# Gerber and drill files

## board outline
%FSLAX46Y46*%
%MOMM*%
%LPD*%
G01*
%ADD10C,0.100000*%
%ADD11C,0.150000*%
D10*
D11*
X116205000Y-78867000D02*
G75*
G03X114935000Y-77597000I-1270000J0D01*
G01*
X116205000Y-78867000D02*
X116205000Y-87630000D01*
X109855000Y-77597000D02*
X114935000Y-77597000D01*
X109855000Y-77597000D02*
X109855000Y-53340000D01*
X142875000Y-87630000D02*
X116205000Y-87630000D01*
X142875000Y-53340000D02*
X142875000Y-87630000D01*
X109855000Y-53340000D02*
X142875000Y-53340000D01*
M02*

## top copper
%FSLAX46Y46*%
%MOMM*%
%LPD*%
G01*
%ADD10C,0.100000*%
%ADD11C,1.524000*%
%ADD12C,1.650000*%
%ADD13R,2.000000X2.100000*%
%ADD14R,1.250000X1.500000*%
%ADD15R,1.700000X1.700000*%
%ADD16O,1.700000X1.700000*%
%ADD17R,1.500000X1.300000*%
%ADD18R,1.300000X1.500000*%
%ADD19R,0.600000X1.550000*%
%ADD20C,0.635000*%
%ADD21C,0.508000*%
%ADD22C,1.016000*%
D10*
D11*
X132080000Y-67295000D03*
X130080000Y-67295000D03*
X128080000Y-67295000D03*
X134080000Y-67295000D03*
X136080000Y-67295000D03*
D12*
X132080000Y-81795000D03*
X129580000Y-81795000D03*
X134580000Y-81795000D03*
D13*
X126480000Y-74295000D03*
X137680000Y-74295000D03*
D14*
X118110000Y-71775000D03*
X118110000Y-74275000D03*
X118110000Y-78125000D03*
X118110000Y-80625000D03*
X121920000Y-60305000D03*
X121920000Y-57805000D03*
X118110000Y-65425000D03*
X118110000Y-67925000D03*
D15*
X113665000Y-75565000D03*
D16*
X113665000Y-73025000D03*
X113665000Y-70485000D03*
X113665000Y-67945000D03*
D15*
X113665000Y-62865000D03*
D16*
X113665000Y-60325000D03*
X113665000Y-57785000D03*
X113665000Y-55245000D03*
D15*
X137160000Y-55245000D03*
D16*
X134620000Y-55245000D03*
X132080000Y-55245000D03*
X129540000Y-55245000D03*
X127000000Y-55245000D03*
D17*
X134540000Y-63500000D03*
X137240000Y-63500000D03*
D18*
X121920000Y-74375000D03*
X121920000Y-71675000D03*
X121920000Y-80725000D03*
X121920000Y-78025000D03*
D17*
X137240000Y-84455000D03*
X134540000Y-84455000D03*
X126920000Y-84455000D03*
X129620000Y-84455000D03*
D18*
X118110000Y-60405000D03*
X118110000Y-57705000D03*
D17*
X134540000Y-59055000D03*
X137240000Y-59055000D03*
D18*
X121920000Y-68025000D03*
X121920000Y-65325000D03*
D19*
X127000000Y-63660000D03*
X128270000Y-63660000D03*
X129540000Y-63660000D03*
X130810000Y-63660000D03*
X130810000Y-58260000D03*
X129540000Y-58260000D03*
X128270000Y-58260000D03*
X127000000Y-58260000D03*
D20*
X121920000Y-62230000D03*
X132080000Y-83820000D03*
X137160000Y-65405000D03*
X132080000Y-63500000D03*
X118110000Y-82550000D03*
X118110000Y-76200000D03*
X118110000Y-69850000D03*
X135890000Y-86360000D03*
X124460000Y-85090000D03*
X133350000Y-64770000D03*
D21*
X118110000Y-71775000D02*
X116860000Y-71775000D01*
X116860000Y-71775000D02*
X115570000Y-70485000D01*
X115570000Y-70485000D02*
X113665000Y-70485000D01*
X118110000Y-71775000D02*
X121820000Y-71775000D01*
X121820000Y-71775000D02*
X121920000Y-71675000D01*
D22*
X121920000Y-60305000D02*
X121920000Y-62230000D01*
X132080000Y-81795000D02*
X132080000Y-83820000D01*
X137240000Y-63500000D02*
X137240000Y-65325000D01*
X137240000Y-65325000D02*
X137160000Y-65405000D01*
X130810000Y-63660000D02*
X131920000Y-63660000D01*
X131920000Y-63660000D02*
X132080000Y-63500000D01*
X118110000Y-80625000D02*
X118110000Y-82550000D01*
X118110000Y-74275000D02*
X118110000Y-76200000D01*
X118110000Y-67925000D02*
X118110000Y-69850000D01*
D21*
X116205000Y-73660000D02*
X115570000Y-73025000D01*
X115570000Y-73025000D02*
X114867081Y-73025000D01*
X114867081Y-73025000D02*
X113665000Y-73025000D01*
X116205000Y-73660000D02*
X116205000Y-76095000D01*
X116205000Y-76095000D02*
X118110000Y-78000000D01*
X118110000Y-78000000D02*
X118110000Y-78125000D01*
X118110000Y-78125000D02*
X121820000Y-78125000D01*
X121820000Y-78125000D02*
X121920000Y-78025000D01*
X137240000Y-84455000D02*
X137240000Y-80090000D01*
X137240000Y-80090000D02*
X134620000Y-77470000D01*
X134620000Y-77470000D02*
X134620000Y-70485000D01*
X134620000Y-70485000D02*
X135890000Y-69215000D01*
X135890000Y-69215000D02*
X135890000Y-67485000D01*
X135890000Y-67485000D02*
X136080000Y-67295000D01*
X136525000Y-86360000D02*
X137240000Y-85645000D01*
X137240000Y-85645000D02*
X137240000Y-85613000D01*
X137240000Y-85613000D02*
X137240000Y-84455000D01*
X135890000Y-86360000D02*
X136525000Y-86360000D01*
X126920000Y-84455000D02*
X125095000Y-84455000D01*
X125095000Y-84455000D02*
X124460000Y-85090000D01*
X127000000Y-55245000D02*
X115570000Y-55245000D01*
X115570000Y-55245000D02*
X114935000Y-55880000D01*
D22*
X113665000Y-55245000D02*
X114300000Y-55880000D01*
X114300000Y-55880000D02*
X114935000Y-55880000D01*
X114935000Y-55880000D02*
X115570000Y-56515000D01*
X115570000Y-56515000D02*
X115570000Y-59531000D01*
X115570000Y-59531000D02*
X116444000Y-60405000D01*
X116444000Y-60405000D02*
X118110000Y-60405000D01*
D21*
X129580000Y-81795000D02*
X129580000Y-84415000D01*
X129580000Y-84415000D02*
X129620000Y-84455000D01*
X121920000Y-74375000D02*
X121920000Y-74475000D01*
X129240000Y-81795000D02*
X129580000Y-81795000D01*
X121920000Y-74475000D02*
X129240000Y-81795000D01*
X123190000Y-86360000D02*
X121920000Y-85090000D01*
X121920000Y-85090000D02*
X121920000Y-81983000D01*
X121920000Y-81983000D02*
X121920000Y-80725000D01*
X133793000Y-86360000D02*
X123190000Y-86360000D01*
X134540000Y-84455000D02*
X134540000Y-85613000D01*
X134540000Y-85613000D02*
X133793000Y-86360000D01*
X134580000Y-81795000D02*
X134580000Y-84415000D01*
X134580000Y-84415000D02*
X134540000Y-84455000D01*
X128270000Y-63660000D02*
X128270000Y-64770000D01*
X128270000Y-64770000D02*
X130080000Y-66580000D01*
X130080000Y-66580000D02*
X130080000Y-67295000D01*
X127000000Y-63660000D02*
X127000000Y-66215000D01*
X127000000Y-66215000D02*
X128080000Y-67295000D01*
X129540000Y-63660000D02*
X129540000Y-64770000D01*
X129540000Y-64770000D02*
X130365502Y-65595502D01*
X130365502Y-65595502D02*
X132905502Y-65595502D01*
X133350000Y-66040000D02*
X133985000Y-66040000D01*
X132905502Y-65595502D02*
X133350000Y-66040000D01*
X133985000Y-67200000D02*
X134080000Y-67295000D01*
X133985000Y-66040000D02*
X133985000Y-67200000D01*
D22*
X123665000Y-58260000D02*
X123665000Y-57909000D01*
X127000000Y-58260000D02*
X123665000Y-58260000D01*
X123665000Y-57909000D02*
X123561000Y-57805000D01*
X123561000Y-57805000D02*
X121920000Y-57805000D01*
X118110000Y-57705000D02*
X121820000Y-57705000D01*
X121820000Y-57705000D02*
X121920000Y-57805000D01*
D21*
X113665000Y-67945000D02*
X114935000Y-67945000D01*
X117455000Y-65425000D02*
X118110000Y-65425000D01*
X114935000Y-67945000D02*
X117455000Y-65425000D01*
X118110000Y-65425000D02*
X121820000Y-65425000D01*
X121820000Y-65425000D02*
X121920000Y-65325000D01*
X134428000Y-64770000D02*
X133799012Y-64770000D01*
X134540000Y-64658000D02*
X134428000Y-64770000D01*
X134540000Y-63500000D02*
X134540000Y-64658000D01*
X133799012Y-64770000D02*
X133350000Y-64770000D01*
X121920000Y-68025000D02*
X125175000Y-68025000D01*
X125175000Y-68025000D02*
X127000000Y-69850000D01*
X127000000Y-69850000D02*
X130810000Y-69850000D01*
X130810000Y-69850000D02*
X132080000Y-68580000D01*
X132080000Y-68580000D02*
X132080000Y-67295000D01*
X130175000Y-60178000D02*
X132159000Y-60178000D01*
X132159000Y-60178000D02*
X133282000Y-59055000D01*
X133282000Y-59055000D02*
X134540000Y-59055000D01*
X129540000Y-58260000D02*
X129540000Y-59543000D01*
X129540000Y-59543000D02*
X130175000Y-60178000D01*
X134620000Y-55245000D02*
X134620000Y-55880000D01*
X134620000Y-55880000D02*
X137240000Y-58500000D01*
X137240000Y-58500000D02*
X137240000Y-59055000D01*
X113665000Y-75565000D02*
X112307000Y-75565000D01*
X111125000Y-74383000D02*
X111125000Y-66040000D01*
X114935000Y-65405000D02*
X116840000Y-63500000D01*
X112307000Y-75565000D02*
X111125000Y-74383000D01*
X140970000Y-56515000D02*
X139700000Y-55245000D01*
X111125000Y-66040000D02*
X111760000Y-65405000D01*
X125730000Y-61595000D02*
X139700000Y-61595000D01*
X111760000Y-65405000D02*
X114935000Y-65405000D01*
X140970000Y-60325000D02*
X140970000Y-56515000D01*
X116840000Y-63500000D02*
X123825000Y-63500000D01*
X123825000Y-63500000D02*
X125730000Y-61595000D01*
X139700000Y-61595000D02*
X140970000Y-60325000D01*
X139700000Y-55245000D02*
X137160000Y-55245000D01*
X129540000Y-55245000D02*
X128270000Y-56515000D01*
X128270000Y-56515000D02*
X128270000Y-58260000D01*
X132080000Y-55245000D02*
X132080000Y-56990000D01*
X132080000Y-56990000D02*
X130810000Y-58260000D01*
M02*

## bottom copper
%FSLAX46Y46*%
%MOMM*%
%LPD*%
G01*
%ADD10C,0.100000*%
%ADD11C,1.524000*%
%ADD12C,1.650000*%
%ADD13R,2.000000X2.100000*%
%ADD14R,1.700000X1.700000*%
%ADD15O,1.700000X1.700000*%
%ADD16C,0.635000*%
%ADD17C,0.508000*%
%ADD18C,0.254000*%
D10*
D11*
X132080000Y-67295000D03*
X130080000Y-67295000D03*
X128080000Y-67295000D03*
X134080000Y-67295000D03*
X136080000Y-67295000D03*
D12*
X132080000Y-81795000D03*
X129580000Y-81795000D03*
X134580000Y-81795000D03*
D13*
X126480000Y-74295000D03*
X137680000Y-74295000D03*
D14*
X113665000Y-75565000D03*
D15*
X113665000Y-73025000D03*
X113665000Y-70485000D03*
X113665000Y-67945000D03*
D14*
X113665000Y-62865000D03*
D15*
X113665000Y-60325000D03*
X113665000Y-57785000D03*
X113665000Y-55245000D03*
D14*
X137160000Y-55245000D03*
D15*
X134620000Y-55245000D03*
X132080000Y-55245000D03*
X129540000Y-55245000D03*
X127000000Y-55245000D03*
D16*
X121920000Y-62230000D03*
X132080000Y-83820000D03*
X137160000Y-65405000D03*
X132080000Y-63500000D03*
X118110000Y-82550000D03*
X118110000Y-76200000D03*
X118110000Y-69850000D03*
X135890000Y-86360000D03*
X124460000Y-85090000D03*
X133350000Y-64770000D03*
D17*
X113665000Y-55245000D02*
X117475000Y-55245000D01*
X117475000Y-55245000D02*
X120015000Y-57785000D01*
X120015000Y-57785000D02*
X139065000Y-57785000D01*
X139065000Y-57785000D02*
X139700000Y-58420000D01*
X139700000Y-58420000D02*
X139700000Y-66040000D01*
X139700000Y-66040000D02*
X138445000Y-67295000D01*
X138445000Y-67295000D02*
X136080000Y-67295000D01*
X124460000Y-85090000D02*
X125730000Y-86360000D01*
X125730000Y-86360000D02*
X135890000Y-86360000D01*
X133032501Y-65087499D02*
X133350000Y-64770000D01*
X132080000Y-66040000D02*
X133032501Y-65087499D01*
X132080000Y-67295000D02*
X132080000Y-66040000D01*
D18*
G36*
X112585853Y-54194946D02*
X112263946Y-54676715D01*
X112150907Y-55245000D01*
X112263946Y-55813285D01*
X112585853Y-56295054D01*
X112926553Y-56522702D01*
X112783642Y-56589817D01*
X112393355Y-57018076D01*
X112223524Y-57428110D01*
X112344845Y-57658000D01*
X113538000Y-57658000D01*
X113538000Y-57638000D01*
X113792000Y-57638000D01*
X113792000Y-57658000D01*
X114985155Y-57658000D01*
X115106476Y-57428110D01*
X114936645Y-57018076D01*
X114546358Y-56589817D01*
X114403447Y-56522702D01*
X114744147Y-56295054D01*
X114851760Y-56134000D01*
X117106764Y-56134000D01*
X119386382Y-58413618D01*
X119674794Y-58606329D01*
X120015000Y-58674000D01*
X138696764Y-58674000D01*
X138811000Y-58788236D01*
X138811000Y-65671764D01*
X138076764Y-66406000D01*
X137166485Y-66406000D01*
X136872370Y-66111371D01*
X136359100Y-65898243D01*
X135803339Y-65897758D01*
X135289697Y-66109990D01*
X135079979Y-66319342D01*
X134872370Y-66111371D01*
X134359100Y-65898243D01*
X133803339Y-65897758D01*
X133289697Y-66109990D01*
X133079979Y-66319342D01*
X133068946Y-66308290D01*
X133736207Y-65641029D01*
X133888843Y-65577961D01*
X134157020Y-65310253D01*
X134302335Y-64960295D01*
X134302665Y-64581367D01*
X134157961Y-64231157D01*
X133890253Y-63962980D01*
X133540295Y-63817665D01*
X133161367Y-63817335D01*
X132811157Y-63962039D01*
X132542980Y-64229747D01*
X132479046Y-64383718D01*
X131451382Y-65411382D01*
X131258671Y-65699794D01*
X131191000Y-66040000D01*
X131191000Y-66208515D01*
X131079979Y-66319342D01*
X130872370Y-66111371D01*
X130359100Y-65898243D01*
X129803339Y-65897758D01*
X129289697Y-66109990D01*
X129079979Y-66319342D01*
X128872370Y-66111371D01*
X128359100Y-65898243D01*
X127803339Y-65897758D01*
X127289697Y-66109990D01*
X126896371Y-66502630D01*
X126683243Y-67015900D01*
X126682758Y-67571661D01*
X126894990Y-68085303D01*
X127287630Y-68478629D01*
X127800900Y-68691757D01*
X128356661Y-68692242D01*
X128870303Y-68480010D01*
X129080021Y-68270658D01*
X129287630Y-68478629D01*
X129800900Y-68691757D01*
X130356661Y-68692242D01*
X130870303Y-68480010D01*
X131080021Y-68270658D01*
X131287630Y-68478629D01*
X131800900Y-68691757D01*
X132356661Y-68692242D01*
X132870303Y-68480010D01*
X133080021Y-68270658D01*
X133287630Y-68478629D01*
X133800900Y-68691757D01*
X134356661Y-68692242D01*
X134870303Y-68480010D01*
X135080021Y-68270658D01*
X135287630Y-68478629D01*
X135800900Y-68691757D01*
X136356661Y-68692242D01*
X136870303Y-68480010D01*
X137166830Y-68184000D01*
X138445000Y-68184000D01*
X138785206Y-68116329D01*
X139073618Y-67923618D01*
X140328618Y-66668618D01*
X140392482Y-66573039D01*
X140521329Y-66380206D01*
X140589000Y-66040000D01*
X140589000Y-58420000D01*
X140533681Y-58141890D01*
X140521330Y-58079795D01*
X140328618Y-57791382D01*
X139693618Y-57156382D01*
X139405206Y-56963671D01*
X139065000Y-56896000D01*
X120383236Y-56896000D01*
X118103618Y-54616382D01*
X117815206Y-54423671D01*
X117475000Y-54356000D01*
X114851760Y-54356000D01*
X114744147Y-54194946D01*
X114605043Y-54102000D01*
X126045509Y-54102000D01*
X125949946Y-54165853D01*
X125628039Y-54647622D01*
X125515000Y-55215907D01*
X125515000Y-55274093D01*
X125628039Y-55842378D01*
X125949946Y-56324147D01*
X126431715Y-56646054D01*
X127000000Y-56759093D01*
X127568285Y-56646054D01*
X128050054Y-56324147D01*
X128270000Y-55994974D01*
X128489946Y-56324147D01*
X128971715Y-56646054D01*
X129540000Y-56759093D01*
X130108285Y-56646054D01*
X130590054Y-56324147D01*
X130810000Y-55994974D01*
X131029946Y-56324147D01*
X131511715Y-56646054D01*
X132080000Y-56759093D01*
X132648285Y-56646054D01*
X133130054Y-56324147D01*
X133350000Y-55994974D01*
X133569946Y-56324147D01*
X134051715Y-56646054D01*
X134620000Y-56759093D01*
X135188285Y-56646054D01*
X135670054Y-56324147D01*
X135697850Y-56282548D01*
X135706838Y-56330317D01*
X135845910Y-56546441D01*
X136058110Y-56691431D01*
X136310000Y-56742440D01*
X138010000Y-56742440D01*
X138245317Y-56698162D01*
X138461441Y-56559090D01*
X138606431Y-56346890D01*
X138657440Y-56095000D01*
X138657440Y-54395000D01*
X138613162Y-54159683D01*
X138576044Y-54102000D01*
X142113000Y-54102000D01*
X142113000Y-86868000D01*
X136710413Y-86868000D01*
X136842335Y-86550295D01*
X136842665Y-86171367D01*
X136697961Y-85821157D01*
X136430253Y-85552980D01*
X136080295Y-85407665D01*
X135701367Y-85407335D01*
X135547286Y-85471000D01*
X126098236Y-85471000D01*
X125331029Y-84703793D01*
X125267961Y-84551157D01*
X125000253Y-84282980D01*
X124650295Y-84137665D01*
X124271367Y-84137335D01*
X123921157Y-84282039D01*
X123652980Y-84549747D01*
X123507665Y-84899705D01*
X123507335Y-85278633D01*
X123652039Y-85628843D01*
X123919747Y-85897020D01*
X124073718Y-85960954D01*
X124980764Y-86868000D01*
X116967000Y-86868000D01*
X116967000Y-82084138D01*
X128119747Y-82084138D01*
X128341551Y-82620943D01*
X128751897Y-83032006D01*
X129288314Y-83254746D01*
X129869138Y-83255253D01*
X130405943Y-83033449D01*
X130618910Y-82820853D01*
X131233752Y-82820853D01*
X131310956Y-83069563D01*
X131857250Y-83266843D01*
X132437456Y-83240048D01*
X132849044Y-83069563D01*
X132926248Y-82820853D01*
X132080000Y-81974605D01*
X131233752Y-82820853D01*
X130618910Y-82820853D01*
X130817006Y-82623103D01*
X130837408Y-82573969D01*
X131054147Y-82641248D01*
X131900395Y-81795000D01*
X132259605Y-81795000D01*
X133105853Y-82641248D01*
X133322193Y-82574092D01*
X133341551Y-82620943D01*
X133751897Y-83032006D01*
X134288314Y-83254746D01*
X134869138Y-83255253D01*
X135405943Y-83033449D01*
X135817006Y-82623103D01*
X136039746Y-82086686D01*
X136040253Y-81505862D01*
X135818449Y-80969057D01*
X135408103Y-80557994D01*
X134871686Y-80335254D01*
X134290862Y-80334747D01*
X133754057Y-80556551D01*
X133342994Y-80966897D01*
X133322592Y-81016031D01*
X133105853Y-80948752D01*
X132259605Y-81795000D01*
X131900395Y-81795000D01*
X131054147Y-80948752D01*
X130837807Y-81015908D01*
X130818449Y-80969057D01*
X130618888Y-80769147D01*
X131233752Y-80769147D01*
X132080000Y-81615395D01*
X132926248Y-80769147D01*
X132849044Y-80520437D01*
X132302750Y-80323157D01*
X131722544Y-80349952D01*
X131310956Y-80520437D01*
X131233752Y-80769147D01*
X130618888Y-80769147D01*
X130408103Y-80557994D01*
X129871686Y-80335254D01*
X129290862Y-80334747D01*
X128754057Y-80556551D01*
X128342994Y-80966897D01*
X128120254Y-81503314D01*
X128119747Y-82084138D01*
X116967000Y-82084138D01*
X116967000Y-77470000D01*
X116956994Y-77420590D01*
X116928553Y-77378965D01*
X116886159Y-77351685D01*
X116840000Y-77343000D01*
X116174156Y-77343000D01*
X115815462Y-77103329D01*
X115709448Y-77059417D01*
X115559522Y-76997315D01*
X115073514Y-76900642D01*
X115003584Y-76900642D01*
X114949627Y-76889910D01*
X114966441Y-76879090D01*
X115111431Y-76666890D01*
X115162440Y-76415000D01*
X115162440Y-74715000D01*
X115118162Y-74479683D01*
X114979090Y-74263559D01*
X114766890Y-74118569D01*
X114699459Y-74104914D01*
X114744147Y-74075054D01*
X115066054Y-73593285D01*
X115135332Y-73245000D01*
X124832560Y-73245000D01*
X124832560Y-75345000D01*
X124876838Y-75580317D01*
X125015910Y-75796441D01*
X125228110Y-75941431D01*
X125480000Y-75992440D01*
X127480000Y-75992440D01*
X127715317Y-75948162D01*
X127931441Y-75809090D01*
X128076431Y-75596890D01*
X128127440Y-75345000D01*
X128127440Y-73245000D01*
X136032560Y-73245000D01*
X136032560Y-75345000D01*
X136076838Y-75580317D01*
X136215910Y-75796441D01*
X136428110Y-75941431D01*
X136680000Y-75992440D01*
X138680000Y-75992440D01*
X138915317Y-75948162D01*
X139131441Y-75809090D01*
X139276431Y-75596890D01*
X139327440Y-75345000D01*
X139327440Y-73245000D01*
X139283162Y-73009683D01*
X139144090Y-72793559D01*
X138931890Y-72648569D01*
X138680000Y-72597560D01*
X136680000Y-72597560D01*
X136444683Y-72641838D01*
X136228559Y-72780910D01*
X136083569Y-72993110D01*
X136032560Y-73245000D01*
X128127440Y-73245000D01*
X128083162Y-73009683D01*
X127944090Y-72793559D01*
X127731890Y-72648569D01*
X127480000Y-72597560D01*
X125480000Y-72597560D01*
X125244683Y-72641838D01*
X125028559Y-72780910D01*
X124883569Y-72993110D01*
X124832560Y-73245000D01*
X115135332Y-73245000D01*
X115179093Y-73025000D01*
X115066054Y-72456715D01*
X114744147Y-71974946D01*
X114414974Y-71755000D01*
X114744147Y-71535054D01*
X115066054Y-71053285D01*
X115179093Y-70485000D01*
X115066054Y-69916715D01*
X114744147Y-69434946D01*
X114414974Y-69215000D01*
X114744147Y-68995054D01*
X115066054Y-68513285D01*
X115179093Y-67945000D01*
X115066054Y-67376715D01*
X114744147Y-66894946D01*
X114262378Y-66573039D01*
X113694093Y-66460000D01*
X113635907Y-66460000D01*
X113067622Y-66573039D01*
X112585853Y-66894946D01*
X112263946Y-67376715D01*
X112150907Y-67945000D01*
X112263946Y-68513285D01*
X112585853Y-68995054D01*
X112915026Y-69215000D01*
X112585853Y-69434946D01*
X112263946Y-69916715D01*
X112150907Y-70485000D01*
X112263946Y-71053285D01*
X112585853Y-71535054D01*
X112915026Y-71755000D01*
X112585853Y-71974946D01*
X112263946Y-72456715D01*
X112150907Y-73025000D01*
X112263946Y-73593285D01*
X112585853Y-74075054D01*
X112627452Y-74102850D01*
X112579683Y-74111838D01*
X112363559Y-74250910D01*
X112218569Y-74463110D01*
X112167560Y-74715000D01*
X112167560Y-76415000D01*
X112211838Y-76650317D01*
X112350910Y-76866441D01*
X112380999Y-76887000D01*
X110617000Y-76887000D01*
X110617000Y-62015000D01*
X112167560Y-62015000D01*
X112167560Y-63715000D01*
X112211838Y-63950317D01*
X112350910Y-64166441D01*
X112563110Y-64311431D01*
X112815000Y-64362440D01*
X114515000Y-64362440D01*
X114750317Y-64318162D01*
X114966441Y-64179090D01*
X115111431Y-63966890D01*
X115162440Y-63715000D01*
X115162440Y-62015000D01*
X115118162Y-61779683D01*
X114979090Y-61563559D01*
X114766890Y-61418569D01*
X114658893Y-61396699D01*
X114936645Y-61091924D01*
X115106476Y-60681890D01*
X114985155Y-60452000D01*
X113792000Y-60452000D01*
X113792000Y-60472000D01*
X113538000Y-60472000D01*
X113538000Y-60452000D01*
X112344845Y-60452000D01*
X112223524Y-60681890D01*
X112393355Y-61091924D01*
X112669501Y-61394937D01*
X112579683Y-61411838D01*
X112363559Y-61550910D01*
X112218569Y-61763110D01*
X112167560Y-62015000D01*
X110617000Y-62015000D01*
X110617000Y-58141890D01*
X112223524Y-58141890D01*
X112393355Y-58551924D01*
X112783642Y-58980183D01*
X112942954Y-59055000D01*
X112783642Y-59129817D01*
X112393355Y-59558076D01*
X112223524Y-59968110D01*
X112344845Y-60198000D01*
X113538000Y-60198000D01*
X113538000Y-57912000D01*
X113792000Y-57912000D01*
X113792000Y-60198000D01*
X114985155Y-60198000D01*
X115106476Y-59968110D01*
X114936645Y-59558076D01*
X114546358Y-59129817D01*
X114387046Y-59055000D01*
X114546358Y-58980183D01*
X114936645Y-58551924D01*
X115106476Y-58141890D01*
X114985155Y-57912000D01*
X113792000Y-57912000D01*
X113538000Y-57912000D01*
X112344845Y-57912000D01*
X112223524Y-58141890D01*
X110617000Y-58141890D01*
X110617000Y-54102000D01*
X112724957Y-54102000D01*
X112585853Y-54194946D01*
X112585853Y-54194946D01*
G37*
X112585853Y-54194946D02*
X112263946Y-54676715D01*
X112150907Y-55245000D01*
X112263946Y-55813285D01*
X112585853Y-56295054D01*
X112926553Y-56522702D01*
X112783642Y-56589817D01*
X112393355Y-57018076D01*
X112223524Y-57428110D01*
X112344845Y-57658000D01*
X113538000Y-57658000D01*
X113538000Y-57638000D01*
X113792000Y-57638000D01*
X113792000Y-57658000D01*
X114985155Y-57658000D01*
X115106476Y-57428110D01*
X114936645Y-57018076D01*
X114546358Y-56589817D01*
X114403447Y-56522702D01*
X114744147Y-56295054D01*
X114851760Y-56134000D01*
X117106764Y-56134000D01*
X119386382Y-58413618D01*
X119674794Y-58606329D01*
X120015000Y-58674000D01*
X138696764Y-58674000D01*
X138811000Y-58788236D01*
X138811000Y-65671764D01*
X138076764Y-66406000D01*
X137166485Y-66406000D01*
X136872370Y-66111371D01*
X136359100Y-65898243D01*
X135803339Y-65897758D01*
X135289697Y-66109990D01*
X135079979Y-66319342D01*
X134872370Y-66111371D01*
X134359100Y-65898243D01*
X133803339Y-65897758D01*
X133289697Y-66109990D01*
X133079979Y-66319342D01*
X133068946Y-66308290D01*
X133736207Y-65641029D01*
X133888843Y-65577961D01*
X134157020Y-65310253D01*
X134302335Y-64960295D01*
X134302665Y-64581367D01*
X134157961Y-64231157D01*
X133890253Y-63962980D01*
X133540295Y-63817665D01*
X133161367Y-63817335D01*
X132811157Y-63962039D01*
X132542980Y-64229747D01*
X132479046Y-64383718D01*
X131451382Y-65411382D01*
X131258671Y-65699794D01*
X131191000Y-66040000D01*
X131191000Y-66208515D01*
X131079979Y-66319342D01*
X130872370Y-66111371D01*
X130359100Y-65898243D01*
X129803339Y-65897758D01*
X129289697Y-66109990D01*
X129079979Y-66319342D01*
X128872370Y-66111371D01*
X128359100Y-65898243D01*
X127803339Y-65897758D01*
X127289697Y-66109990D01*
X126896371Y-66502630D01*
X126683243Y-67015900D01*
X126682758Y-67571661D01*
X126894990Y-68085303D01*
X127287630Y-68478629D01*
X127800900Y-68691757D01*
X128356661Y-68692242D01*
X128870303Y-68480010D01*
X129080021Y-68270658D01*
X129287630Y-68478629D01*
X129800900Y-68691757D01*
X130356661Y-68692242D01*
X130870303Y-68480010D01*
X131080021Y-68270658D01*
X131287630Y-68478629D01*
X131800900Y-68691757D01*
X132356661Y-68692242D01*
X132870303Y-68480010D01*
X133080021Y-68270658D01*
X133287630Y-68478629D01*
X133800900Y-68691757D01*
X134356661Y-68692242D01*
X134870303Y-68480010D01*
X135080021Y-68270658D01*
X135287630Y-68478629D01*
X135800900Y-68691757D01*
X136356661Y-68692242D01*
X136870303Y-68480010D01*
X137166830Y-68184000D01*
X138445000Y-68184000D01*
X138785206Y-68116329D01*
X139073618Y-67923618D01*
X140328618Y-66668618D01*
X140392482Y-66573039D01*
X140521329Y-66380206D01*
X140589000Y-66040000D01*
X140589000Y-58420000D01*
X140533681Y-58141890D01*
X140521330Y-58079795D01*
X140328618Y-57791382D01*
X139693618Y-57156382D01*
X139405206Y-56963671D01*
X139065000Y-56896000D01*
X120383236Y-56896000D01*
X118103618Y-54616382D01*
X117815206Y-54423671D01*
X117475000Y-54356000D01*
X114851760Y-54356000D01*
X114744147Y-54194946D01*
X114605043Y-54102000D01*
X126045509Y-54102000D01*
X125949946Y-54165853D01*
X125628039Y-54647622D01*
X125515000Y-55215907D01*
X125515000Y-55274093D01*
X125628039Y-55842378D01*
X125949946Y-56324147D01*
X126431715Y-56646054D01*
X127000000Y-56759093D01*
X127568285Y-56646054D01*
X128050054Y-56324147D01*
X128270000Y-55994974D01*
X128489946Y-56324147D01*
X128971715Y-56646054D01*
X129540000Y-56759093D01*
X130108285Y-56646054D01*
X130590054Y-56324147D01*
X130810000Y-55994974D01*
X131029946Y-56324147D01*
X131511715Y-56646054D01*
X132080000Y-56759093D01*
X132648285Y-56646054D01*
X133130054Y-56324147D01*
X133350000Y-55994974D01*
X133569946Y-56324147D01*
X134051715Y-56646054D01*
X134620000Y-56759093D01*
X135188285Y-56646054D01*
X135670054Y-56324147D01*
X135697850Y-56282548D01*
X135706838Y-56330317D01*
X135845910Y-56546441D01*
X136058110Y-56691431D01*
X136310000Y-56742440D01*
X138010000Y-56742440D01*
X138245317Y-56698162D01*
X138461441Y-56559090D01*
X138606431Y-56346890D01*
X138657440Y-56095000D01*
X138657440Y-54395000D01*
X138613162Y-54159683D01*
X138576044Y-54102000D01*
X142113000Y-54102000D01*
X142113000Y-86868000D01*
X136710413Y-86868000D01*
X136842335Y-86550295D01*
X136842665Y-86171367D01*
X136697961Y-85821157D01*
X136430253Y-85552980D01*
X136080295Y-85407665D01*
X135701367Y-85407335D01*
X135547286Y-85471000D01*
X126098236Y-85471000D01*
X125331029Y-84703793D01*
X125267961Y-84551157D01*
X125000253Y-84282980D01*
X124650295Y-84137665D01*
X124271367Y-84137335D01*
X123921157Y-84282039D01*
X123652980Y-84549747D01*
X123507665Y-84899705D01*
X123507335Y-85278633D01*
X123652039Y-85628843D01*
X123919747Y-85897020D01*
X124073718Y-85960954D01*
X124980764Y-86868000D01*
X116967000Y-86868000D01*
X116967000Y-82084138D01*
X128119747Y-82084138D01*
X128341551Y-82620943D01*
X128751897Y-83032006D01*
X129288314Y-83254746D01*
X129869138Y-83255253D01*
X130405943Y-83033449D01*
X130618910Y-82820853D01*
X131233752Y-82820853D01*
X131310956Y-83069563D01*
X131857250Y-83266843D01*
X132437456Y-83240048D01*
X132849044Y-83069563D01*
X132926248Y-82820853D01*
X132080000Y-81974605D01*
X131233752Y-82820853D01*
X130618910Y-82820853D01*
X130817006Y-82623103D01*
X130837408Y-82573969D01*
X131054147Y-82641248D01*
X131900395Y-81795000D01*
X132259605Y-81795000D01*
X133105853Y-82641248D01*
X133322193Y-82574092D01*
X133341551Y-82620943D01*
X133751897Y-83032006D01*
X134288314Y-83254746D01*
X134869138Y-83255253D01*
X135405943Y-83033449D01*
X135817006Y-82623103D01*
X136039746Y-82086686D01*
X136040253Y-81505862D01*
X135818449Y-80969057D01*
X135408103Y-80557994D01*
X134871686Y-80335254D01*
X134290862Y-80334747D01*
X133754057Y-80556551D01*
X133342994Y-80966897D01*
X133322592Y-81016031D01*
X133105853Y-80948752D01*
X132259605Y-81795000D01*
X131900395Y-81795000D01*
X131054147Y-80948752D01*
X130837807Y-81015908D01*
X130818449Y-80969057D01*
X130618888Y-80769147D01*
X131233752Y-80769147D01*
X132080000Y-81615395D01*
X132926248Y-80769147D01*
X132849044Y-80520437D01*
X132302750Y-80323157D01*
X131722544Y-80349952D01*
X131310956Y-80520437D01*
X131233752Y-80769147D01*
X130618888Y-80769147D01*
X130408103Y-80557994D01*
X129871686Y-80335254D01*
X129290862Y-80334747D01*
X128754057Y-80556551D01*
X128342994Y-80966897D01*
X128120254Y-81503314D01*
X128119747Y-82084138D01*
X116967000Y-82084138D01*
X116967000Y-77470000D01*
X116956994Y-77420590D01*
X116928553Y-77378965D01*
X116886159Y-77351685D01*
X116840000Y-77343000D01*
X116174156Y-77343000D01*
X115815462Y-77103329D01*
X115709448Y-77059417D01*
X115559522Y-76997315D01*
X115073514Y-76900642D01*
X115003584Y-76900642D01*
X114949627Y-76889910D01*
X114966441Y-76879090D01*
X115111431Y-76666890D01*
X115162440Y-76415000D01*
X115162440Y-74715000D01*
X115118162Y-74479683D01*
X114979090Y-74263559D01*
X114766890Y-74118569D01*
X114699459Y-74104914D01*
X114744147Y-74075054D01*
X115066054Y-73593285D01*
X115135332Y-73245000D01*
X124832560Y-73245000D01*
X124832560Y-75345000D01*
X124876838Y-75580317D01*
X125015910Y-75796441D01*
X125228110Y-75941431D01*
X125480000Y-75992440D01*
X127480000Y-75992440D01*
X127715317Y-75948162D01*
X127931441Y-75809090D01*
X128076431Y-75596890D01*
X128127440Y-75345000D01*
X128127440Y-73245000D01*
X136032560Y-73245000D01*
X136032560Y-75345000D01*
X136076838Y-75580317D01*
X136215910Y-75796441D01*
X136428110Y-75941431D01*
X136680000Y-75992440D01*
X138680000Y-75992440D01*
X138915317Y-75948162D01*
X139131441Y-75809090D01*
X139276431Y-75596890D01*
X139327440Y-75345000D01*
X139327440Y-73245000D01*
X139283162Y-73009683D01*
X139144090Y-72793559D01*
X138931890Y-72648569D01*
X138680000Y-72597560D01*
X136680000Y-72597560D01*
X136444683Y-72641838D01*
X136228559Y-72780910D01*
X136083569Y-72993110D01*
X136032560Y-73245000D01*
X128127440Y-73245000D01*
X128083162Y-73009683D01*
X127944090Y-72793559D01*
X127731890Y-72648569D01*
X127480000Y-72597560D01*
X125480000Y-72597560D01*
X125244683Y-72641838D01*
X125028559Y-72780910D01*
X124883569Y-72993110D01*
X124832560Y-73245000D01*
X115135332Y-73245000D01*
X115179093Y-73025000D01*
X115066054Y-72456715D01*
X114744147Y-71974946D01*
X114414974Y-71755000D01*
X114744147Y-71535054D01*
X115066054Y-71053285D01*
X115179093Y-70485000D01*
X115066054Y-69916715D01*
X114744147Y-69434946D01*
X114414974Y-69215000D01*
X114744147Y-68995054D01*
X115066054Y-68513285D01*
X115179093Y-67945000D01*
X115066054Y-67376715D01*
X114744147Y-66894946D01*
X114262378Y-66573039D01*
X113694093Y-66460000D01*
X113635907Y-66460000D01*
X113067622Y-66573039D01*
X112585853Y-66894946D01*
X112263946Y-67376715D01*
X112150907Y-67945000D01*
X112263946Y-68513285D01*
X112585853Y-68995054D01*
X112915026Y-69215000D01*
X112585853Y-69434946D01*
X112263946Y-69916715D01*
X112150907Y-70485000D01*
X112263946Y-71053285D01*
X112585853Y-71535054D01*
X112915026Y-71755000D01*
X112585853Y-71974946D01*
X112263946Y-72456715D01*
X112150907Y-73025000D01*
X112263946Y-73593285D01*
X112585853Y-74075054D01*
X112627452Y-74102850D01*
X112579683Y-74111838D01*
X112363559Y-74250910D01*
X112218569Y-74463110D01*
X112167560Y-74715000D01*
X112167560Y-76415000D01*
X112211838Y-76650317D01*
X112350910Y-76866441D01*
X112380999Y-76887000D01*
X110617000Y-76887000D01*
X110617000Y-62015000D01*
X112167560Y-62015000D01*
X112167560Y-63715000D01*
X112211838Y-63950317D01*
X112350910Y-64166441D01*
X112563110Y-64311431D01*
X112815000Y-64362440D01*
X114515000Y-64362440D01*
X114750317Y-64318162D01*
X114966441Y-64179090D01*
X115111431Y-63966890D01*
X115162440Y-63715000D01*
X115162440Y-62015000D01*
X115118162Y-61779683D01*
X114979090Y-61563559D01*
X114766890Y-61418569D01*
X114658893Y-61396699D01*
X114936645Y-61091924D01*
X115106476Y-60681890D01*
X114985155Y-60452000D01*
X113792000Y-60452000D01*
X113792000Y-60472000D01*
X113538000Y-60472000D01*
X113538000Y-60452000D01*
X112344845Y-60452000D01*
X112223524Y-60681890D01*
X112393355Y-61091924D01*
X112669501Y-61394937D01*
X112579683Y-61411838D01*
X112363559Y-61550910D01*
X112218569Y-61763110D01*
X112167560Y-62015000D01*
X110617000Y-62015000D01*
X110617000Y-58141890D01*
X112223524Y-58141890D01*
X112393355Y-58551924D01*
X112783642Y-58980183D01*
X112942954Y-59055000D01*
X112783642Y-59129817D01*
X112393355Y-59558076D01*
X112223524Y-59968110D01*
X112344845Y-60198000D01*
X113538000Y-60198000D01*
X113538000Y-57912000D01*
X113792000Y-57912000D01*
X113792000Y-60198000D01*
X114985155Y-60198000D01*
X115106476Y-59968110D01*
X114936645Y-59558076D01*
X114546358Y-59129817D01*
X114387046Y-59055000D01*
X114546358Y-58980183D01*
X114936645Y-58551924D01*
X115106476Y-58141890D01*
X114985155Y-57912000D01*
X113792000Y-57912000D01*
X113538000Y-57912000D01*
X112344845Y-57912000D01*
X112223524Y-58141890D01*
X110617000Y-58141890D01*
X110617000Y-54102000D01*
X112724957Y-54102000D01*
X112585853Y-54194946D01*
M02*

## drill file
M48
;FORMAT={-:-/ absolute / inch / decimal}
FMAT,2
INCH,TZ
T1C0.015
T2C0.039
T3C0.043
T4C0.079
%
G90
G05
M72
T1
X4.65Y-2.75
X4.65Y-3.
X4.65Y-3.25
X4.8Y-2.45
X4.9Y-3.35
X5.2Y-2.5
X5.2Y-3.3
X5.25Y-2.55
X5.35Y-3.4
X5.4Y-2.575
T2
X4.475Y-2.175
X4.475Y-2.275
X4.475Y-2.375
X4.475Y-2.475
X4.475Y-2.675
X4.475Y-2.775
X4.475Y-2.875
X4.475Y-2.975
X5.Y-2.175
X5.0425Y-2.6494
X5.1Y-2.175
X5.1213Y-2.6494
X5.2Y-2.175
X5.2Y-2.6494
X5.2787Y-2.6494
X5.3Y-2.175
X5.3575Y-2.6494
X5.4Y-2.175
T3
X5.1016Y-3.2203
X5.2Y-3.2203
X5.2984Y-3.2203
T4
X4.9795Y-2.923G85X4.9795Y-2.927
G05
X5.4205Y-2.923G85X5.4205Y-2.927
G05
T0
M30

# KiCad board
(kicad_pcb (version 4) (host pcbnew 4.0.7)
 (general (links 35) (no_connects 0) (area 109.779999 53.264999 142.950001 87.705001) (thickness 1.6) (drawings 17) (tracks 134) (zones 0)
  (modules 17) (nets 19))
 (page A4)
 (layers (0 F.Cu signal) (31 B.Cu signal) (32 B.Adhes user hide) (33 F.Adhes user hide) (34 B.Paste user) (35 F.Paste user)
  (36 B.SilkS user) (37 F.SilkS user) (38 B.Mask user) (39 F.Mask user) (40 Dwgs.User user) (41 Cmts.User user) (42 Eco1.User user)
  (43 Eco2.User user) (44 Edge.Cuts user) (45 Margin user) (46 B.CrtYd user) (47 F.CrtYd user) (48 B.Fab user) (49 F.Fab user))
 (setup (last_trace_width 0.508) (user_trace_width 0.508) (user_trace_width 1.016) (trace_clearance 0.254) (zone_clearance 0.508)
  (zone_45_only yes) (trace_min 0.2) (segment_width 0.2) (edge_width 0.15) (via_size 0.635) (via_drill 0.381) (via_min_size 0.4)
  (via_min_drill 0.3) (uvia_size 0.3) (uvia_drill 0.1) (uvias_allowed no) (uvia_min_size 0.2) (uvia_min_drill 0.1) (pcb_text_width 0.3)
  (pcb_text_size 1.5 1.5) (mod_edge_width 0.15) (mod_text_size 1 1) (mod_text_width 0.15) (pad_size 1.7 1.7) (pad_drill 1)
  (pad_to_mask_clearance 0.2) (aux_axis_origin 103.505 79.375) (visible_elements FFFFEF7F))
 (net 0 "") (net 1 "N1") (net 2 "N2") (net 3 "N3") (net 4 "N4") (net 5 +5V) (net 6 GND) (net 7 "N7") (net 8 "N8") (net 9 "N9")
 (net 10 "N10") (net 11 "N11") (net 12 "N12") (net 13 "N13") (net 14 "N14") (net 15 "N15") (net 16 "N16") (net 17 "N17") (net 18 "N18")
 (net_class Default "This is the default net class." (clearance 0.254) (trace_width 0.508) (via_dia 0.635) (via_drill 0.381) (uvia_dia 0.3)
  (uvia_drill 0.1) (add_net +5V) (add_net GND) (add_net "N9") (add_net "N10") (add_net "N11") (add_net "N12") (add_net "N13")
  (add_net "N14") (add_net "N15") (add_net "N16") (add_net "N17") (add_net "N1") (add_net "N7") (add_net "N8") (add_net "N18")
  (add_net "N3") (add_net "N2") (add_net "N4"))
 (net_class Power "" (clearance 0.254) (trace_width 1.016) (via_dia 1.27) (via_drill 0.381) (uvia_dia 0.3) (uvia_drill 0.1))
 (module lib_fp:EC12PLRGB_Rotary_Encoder (layer F.Cu) (at 132.08 74.295)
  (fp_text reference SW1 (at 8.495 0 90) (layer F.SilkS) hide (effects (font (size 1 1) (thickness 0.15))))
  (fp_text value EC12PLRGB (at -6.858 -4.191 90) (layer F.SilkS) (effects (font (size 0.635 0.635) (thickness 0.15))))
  (pad 3 thru_hole circle (at 0 -7) (size 1.524 1.524) (drill 1) (layers *.Cu *.Mask) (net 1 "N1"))
  (pad 2 thru_hole circle (at -2 -7) (size 1.524 1.524) (drill 1) (layers *.Cu *.Mask) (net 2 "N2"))
  (pad 1 thru_hole circle (at -4 -7) (size 1.524 1.524) (drill 1) (layers *.Cu *.Mask) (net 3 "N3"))
  (pad 4 thru_hole circle (at 2 -7) (size 1.524 1.524) (drill 1) (layers *.Cu *.Mask) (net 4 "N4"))
  (pad 5 thru_hole circle (at 4 -7) (size 1.524 1.524) (drill 1) (layers *.Cu *.Mask) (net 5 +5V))
  (pad C thru_hole circle (at 0 7.5) (size 1.65 1.65) (drill 1.1) (layers *.Cu *.Mask) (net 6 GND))
  (pad A thru_hole circle (at -2.5 7.5) (size 1.65 1.65) (drill 1.1) (layers *.Cu *.Mask) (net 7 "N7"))
  (pad B thru_hole circle (at 2.5 7.5) (size 1.65 1.65) (drill 1.1) (layers *.Cu *.Mask) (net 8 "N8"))
  (pad "" np_thru_hole rect (at -5.6 0) (size 2 2.1) (drill oval 2 2.1) (layers *.Cu *.Mask))
  (pad "" np_thru_hole rect (at 5.6 0) (size 2 2.1) (drill oval 2 2.1) (layers *.Cu *.Mask)))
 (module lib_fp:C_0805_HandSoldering (layer F.Cu) (at 118.11 73.025 270)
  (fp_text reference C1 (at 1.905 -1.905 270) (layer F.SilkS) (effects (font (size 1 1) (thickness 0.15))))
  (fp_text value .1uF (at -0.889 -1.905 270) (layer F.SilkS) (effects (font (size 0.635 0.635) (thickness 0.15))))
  (pad 1 smd rect (at -1.25 0 270) (size 1.5 1.25) (layers F.Cu F.Paste F.Mask) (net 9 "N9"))
  (pad 2 smd rect (at 1.25 0 270) (size 1.5 1.25) (layers F.Cu F.Paste F.Mask) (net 6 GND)))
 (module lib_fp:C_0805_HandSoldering (layer F.Cu) (at 118.11 79.375 270)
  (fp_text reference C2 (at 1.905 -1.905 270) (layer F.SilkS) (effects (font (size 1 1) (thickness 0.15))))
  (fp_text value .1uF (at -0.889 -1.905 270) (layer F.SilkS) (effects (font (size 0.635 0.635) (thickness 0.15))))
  (pad 1 smd rect (at -1.25 0 270) (size 1.5 1.25) (layers F.Cu F.Paste F.Mask) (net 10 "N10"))
  (pad 2 smd rect (at 1.25 0 270) (size 1.5 1.25) (layers F.Cu F.Paste F.Mask) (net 6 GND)))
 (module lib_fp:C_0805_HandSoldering (layer F.Cu) (at 121.92 59.055 90)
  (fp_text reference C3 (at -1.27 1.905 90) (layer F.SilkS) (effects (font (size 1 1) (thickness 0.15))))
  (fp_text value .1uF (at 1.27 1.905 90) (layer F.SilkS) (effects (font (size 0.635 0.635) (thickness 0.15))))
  (pad 1 smd rect (at -1.25 0 90) (size 1.5 1.25) (layers F.Cu F.Paste F.Mask) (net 6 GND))
  (pad 2 smd rect (at 1.25 0 90) (size 1.5 1.25) (layers F.Cu F.Paste F.Mask) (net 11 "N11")))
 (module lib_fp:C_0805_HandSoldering (layer F.Cu) (at 118.11 66.675 270)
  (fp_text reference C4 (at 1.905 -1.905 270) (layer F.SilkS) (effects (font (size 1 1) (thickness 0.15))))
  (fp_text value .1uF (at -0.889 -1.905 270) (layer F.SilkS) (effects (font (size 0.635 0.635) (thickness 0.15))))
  (pad 1 smd rect (at -1.25 0 270) (size 1.5 1.25) (layers F.Cu F.Paste F.Mask) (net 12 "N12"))
  (pad 2 smd rect (at 1.25 0 270) (size 1.5 1.25) (layers F.Cu F.Paste F.Mask) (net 6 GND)))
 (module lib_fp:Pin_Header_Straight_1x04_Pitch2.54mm (layer B.Cu) (at 113.665 75.565)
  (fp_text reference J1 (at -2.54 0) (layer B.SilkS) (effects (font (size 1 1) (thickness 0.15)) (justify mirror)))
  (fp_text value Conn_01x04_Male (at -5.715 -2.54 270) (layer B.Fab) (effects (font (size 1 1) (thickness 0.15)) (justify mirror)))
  (pad 1 thru_hole rect (at 0 0) (size 1.7 1.7) (drill 1) (layers *.Cu *.Mask) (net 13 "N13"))
  (pad 2 thru_hole oval (at 0 -2.54) (size 1.7 1.7) (drill 1) (layers *.Cu *.Mask) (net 10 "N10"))
  (pad 3 thru_hole oval (at 0 -5.08) (size 1.7 1.7) (drill 1) (layers *.Cu *.Mask) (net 9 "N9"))
  (pad 4 thru_hole oval (at 0 -7.62) (size 1.7 1.7) (drill 1) (layers *.Cu *.Mask) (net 12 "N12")))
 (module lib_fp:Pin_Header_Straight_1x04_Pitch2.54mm (layer B.Cu) (at 113.665 62.865)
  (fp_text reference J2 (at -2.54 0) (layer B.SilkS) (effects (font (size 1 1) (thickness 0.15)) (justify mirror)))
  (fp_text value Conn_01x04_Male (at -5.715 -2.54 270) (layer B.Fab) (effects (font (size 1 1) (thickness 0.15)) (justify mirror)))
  (pad 1 thru_hole rect (at 0 0) (size 1.7 1.7) (drill 1) (layers *.Cu *.Mask) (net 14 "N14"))
  (pad 2 thru_hole oval (at 0 -2.54) (size 1.7 1.7) (drill 1) (layers *.Cu *.Mask) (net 6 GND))
  (pad 3 thru_hole oval (at 0 -5.08) (size 1.7 1.7) (drill 1) (layers *.Cu *.Mask) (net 6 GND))
  (pad 4 thru_hole oval (at 0 -7.62) (size 1.7 1.7) (drill 1) (layers *.Cu *.Mask) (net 5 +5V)))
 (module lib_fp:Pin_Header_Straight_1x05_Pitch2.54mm (layer F.Cu) (at 137.16 55.245 270)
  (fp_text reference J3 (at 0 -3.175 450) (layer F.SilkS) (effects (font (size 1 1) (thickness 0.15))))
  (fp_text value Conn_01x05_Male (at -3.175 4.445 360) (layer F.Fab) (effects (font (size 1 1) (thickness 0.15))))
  (pad 1 thru_hole rect (at 0 0 270) (size 1.7 1.7) (drill 1) (layers *.Cu *.Mask) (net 13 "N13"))
  (pad 2 thru_hole oval (at 0 2.54 270) (size 1.7 1.7) (drill 1) (layers *.Cu *.Mask) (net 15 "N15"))
  (pad 3 thru_hole oval (at 0 5.08 270) (size 1.7 1.7) (drill 1) (layers *.Cu *.Mask) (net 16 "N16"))
  (pad 4 thru_hole oval (at 0 7.62 270) (size 1.7 1.7) (drill 1) (layers *.Cu *.Mask) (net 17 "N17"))
  (pad 5 thru_hole oval (at 0 10.16 270) (size 1.7 1.7) (drill 1) (layers *.Cu *.Mask) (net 5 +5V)))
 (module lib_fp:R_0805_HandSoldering (layer F.Cu) (at 135.89 63.5)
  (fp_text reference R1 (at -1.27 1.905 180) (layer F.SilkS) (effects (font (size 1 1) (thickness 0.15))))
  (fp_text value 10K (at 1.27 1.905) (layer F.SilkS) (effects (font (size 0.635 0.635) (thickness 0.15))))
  (pad 1 smd rect (at -1.35 0) (size 1.5 1.3) (layers F.Cu F.Paste F.Mask) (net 1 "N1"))
  (pad 2 smd rect (at 1.35 0) (size 1.5 1.3) (layers F.Cu F.Paste F.Mask) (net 6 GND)))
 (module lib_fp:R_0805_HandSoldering (layer F.Cu) (at 121.92 73.025 90)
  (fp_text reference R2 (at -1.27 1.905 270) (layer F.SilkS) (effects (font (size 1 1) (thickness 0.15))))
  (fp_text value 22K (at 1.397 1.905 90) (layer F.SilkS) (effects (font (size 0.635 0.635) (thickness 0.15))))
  (pad 1 smd rect (at -1.35 0 90) (size 1.5 1.3) (layers F.Cu F.Paste F.Mask) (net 7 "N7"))
  (pad 2 smd rect (at 1.35 0 90) (size 1.5 1.3) (layers F.Cu F.Paste F.Mask) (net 9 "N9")))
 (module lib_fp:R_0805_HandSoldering (layer F.Cu) (at 121.92 79.375 90)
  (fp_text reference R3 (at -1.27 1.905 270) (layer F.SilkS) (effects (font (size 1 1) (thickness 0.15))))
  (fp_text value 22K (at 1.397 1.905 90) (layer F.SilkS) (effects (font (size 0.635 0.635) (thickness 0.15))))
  (pad 1 smd rect (at -1.35 0 90) (size 1.5 1.3) (layers F.Cu F.Paste F.Mask) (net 8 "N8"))
  (pad 2 smd rect (at 1.35 0 90) (size 1.5 1.3) (layers F.Cu F.Paste F.Mask) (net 10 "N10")))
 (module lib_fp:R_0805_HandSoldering (layer F.Cu) (at 135.89 84.455 180)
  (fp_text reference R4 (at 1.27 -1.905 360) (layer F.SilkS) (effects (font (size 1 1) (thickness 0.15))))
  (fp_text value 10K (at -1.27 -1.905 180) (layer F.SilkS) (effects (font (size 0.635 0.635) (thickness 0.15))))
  (pad 1 smd rect (at -1.35 0 180) (size 1.5 1.3) (layers F.Cu F.Paste F.Mask) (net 5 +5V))
  (pad 2 smd rect (at 1.35 0 180) (size 1.5 1.3) (layers F.Cu F.Paste F.Mask) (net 8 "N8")))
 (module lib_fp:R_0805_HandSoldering (layer F.Cu) (at 128.27 84.455)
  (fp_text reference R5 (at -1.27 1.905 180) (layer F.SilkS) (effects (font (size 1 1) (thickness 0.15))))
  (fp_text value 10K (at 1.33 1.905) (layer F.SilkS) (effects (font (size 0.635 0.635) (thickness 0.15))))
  (pad 1 smd rect (at -1.35 0) (size 1.5 1.3) (layers F.Cu F.Paste F.Mask) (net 5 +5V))
  (pad 2 smd rect (at 1.35 0) (size 1.5 1.3) (layers F.Cu F.Paste F.Mask) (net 7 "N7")))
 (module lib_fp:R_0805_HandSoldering (layer F.Cu) (at 118.11 59.055 90)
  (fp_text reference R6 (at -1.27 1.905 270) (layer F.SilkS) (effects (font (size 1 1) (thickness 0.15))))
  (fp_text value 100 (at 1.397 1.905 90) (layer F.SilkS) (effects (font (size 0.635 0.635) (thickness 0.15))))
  (pad 1 smd rect (at -1.35 0 90) (size 1.5 1.3) (layers F.Cu F.Paste F.Mask) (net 5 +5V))
  (pad 2 smd rect (at 1.35 0 90) (size 1.5 1.3) (layers F.Cu F.Paste F.Mask) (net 11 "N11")))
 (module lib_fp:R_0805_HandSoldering (layer F.Cu) (at 135.89 59.055)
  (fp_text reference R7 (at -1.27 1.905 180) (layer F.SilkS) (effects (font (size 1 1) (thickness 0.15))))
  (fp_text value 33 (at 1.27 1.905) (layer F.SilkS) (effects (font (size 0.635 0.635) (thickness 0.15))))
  (pad 1 smd rect (at -1.35 0) (size 1.5 1.3) (layers F.Cu F.Paste F.Mask) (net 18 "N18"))
  (pad 2 smd rect (at 1.35 0) (size 1.5 1.3) (layers F.Cu F.Paste F.Mask) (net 15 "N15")))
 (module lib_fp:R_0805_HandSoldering (layer F.Cu) (at 121.92 66.675 90)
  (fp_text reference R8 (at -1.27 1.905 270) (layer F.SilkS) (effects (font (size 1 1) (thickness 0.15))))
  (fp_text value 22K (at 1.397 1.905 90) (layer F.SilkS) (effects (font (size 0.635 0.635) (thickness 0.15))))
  (pad 1 smd rect (at -1.35 0 90) (size 1.5 1.3) (layers F.Cu F.Paste F.Mask) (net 1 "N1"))
  (pad 2 smd rect (at 1.35 0 90) (size 1.5 1.3) (layers F.Cu F.Paste F.Mask) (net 12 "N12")))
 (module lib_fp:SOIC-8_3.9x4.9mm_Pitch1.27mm (layer F.Cu) (at 128.905 60.96 90)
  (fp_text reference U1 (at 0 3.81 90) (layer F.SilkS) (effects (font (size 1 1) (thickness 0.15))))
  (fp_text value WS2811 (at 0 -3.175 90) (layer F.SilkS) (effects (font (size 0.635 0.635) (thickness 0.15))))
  (pad 1 smd rect (at -2.7 -1.905 90) (size 1.55 0.6) (layers F.Cu F.Paste F.Mask) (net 3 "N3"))
  (pad 2 smd rect (at -2.7 -0.635 90) (size 1.55 0.6) (layers F.Cu F.Paste F.Mask) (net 2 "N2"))
  (pad 3 smd rect (at -2.7 0.635 90) (size 1.55 0.6) (layers F.Cu F.Paste F.Mask) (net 4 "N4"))
  (pad 4 smd rect (at -2.7 1.905 90) (size 1.55 0.6) (layers F.Cu F.Paste F.Mask) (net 6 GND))
  (pad 5 smd rect (at 2.7 1.905 90) (size 1.55 0.6) (layers F.Cu F.Paste F.Mask) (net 16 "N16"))
  (pad 6 smd rect (at 2.7 0.635 90) (size 1.55 0.6) (layers F.Cu F.Paste F.Mask) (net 18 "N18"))
  (pad 7 smd rect (at 2.7 -0.635 90) (size 1.55 0.6) (layers F.Cu F.Paste F.Mask) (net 17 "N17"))
  (pad 8 smd rect (at 2.7 -1.905 90) (size 1.55 0.6) (layers F.Cu F.Paste F.Mask) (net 11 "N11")))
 (gr_arc (start 114.935 78.867) (end 114.935 77.597) (angle 90) (layer Edge.Cuts) (width 0.15))
 (gr_line (start 116.205 78.867) (end 116.205 87.63) (layer Edge.Cuts) (width 0.15))
 (gr_line (start 109.855 77.597) (end 114.935 77.597) (layer Edge.Cuts) (width 0.15))
 (gr_line (start 109.855 77.597) (end 109.855 53.34) (layer Edge.Cuts) (width 0.15))
 (gr_line (start 142.875 87.63) (end 116.205 87.63) (layer Edge.Cuts) (width 0.15))
 (gr_line (start 142.875 53.34) (end 142.875 87.63) (layer Edge.Cuts) (width 0.15))
 (gr_line (start 109.855 53.34) (end 142.875 53.34) (layer Edge.Cuts) (width 0.15))
 (segment (start 118.11 71.775) (end 116.86 71.775) (width 0.508) (layer F.Cu) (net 9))
 (segment (start 116.86 71.775) (end 115.57 70.485) (width 0.508) (layer F.Cu) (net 9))
 (segment (start 115.57 70.485) (end 113.665 70.485) (width 0.508) (layer F.Cu) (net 9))
 (segment (start 118.11 71.775) (end 121.82 71.775) (width 0.508) (layer F.Cu) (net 9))
 (segment (start 121.82 71.775) (end 121.92 71.675) (width 0.508) (layer F.Cu) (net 9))
 (segment (start 121.92 60.305) (end 121.92 62.23) (width 1.016) (layer F.Cu) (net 6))
 (via (at 121.92 62.23) (size 0.635) (drill 0.381) (layers F.Cu B.Cu) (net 6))
 (segment (start 132.08 81.795) (end 132.08 83.82) (width 1.016) (layer F.Cu) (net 6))
 (via (at 132.08 83.82) (size 0.635) (drill 0.381) (layers F.Cu B.Cu) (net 6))
 (segment (start 137.24 63.5) (end 137.24 65.325) (width 1.016) (layer F.Cu) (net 6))
 (segment (start 137.24 65.325) (end 137.16 65.405) (width 1.016) (layer F.Cu) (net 6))
 (via (at 137.16 65.405) (size 0.635) (drill 0.381) (layers F.Cu B.Cu) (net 6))
 (segment (start 130.81 63.66) (end 131.92 63.66) (width 1.016) (layer F.Cu) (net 6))
 (segment (start 131.92 63.66) (end 132.08 63.5) (width 1.016) (layer F.Cu) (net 6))
 (via (at 132.08 63.5) (size 0.635) (drill 0.381) (layers F.Cu B.Cu) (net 6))
 (segment (start 118.11 80.625) (end 118.11 82.55) (width 1.016) (layer F.Cu) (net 6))
 (via (at 118.11 82.55) (size 0.635) (drill 0.381) (layers F.Cu B.Cu) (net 6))
 (segment (start 118.11 74.275) (end 118.11 76.2) (width 1.016) (layer F.Cu) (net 6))
 (via (at 118.11 76.2) (size 0.635) (drill 0.381) (layers F.Cu B.Cu) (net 6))
 (via (at 118.11 69.85) (size 0.635) (drill 0.381) (layers F.Cu B.Cu) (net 6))
 (segment (start 118.11 67.925) (end 118.11 69.85) (width 1.016) (layer F.Cu) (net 6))
 (segment (start 116.205 73.66) (end 115.57 73.025) (width 0.508) (layer F.Cu) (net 10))
 (segment (start 115.57 73.025) (end 114.867081 73.025) (width 0.508) (layer F.Cu) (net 10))
 (segment (start 114.867081 73.025) (end 113.665 73.025) (width 0.508) (layer F.Cu) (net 10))
 (segment (start 116.205 73.66) (end 116.205 76.095) (width 0.508) (layer F.Cu) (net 10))
 (segment (start 116.205 76.095) (end 118.11 78) (width 0.508) (layer F.Cu) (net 10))
 (segment (start 118.11 78) (end 118.11 78.125) (width 0.508) (layer F.Cu) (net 10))
 (segment (start 118.11 78.125) (end 121.82 78.125) (width 0.508) (layer F.Cu) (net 10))
 (segment (start 121.82 78.125) (end 121.92 78.025) (width 0.508) (layer F.Cu) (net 10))
 (segment (start 137.24 84.455) (end 137.24 80.09) (width 0.508) (layer F.Cu) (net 5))
 (segment (start 137.24 80.09) (end 134.62 77.47) (width 0.508) (layer F.Cu) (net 5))
 (segment (start 134.62 77.47) (end 134.62 70.485) (width 0.508) (layer F.Cu) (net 5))
 (segment (start 134.62 70.485) (end 135.89 69.215) (width 0.508) (layer F.Cu) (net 5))
 (segment (start 135.89 69.215) (end 135.89 67.485) (width 0.508) (layer F.Cu) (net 5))
 (segment (start 135.89 67.485) (end 136.08 67.295) (width 0.508) (layer F.Cu) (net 5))
 (segment (start 113.665 55.245) (end 117.475 55.245) (width 0.508) (layer B.Cu) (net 5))
 (segment (start 117.475 55.245) (end 120.015 57.785) (width 0.508) (layer B.Cu) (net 5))
 (segment (start 120.015 57.785) (end 139.065 57.785) (width 0.508) (layer B.Cu) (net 5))
 (segment (start 139.065 57.785) (end 139.7 58.42) (width 0.508) (layer B.Cu) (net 5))
 (segment (start 139.7 58.42) (end 139.7 66.04) (width 0.508) (layer B.Cu) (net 5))
 (segment (start 139.7 66.04) (end 138.445 67.295) (width 0.508) (layer B.Cu) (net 5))
 (segment (start 138.445 67.295) (end 136.08 67.295) (width 0.508) (layer B.Cu) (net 5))
 (segment (start 136.525 86.36) (end 137.24 85.645) (width 0.508) (layer F.Cu) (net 5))
 (segment (start 137.24 85.645) (end 137.24 85.613) (width 0.508) (layer F.Cu) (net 5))
 (segment (start 137.24 85.613) (end 137.24 84.455) (width 0.508) (layer F.Cu) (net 5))
 (segment (start 135.89 86.36) (end 136.525 86.36) (width 0.508) (layer F.Cu) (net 5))
 (segment (start 124.46 85.09) (end 125.73 86.36) (width 0.508) (layer B.Cu) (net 5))
 (segment (start 125.73 86.36) (end 135.89 86.36) (width 0.508) (layer B.Cu) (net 5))
 (via (at 135.89 86.36) (size 0.635) (drill 0.381) (layers F.Cu B.Cu) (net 5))
 (segment (start 126.92 84.455) (end 125.095 84.455) (width 0.508) (layer F.Cu) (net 5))
 (segment (start 125.095 84.455) (end 124.46 85.09) (width 0.508) (layer F.Cu) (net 5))
 (via (at 124.46 85.09) (size 0.635) (drill 0.381) (layers F.Cu B.Cu) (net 5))
 (segment (start 127 55.245) (end 115.57 55.245) (width 0.508) (layer F.Cu) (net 5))
 (segment (start 115.57 55.245) (end 114.935 55.88) (width 0.508) (layer F.Cu) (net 5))
 (segment (start 113.665 55.245) (end 114.3 55.88) (width 1.016) (layer F.Cu) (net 5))
 (segment (start 114.3 55.88) (end 114.935 55.88) (width 1.016) (layer F.Cu) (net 5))
 (segment (start 114.935 55.88) (end 115.57 56.515) (width 1.016) (layer F.Cu) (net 5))
 (segment (start 115.57 56.515) (end 115.57 59.531) (width 1.016) (layer F.Cu) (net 5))
 (segment (start 115.57 59.531) (end 116.444 60.405) (width 1.016) (layer F.Cu) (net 5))
 (segment (start 116.444 60.405) (end 118.11 60.405) (width 1.016) (layer F.Cu) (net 5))
 (segment (start 129.58 81.795) (end 129.58 84.415) (width 0.508) (layer F.Cu) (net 7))
 (segment (start 129.58 84.415) (end 129.62 84.455) (width 0.508) (layer F.Cu) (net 7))
 (segment (start 121.92 74.375) (end 121.92 74.475) (width 0.508) (layer F.Cu) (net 7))
 (segment (start 129.24 81.795) (end 129.58 81.795) (width 0.508) (layer F.Cu) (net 7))
 (segment (start 121.92 74.475) (end 129.24 81.795) (width 0.508) (layer F.Cu) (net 7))
 (segment (start 123.19 86.36) (end 121.92 85.09) (width 0.508) (layer F.Cu) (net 8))
 (segment (start 121.92 85.09) (end 121.92 81.983) (width 0.508) (layer F.Cu) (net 8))
 (segment (start 121.92 81.983) (end 121.92 80.725) (width 0.508) (layer F.Cu) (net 8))
 (segment (start 133.793 86.36) (end 123.19 86.36) (width 0.508) (layer F.Cu) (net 8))
 (segment (start 134.54 84.455) (end 134.54 85.613) (width 0.508) (layer F.Cu) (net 8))
 (segment (start 134.54 85.613) (end 133.793 86.36) (width 0.508) (layer F.Cu) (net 8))
 (segment (start 134.58 81.795) (end 134.58 84.415) (width 0.508) (layer F.Cu) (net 8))
 (segment (start 134.58 84.415) (end 134.54 84.455) (width 0.508) (layer F.Cu) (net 8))
 (segment (start 128.27 63.66) (end 128.27 64.77) (width 0.508) (layer F.Cu) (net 2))
 (segment (start 128.27 64.77) (end 130.08 66.58) (width 0.508) (layer F.Cu) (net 2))
 (segment (start 130.08 66.58) (end 130.08 67.295) (width 0.508) (layer F.Cu) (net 2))
 (segment (start 127 63.66) (end 127 66.215) (width 0.508) (layer F.Cu) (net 3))
 (segment (start 127 66.215) (end 128.08 67.295) (width 0.508) (layer F.Cu) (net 3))
 (segment (start 129.54 63.66) (end 129.54 64.77) (width 0.508) (layer F.Cu) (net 4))
 (segment (start 129.54 64.77) (end 130.365502 65.595502) (width 0.508) (layer F.Cu) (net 4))
 (segment (start 130.365502 65.595502) (end 132.905502 65.595502) (width 0.508) (layer F.Cu) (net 4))
 (segment (start 133.35 66.04) (end 133.985 66.04) (width 0.508) (layer F.Cu) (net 4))
 (segment (start 132.905502 65.595502) (end 133.35 66.04) (width 0.508) (layer F.Cu) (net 4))
 (segment (start 133.985 67.2) (end 134.08 67.295) (width 0.508) (layer F.Cu) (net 4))
 (segment (start 133.985 66.04) (end 133.985 67.2) (width 0.508) (layer F.Cu) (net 4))
 (segment (start 123.665 58.26) (end 123.665 57.909) (width 1.016) (layer F.Cu) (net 11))
 (segment (start 127 58.26) (end 123.665 58.26) (width 1.016) (layer F.Cu) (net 11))
 (segment (start 123.665 57.909) (end 123.561 57.805) (width 1.016) (layer F.Cu) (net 11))
 (segment (start 123.561 57.805) (end 121.92 57.805) (width 1.016) (layer F.Cu) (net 11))
 (segment (start 118.11 57.705) (end 121.82 57.705) (width 1.016) (layer F.Cu) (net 11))
 (segment (start 121.82 57.705) (end 121.92 57.805) (width 1.016) (layer F.Cu) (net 11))
 (segment (start 113.665 67.945) (end 114.935 67.945) (width 0.508) (layer F.Cu) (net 12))
 (segment (start 117.455 65.425) (end 118.11 65.425) (width 0.508) (layer F.Cu) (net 12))
 (segment (start 114.935 67.945) (end 117.455 65.425) (width 0.508) (layer F.Cu) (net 12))
 (segment (start 118.11 65.425) (end 121.82 65.425) (width 0.508) (layer F.Cu) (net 12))
 (segment (start 121.82 65.425) (end 121.92 65.325) (width 0.508) (layer F.Cu) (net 12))
 (segment (start 133.032501 65.087499) (end 133.35 64.77) (width 0.508) (layer B.Cu) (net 1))
 (segment (start 132.08 66.04) (end 133.032501 65.087499) (width 0.508) (layer B.Cu) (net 1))
 (segment (start 132.08 67.295) (end 132.08 66.04) (width 0.508) (layer B.Cu) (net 1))
 (segment (start 134.428 64.77) (end 133.799012 64.77) (width 0.508) (layer F.Cu) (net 1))
 (segment (start 134.54 64.658) (end 134.428 64.77) (width 0.508) (layer F.Cu) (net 1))
 (segment (start 134.54 63.5) (end 134.54 64.658) (width 0.508) (layer F.Cu) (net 1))
 (segment (start 133.799012 64.77) (end 133.35 64.77) (width 0.508) (layer F.Cu) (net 1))
 (via (at 133.35 64.77) (size 0.635) (drill 0.381) (layers F.Cu B.Cu) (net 1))
 (segment (start 121.92 68.025) (end 125.175 68.025) (width 0.508) (layer F.Cu) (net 1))
 (segment (start 125.175 68.025) (end 127 69.85) (width 0.508) (layer F.Cu) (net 1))
 (segment (start 127 69.85) (end 130.81 69.85) (width 0.508) (layer F.Cu) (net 1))
 (segment (start 130.81 69.85) (end 132.08 68.58) (width 0.508) (layer F.Cu) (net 1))
 (segment (start 132.08 68.58) (end 132.08 67.295) (width 0.508) (layer F.Cu) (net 1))
 (segment (start 130.175 60.178) (end 132.159 60.178) (width 0.508) (layer F.Cu) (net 18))
 (segment (start 132.159 60.178) (end 133.282 59.055) (width 0.508) (layer F.Cu) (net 18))
 (segment (start 133.282 59.055) (end 134.54 59.055) (width 0.508) (layer F.Cu) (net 18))
 (segment (start 129.54 58.26) (end 129.54 59.543) (width 0.508) (layer F.Cu) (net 18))
 (segment (start 129.54 59.543) (end 130.175 60.178) (width 0.508) (layer F.Cu) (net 18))
 (segment (start 134.62 55.245) (end 134.62 55.88) (width 0.508) (layer F.Cu) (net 15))
 (segment (start 134.62 55.88) (end 137.24 58.5) (width 0.508) (layer F.Cu) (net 15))
 (segment (start 137.24 58.5) (end 137.24 59.055) (width 0.508) (layer F.Cu) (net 15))
 (segment (start 113.665 75.565) (end 112.307 75.565) (width 0.508) (layer F.Cu) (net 13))
 (segment (start 111.125 74.383) (end 111.125 66.04) (width 0.508) (layer F.Cu) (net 13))
 (segment (start 114.935 65.405) (end 116.84 63.5) (width 0.508) (layer F.Cu) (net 13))
 (segment (start 112.307 75.565) (end 111.125 74.383) (width 0.508) (layer F.Cu) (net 13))
 (segment (start 140.97 56.515) (end 139.7 55.245) (width 0.508) (layer F.Cu) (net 13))
 (segment (start 111.125 66.04) (end 111.76 65.405) (width 0.508) (layer F.Cu) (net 13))
 (segment (start 125.73 61.595) (end 139.7 61.595) (width 0.508) (layer F.Cu) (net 13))
 (segment (start 111.76 65.405) (end 114.935 65.405) (width 0.508) (layer F.Cu) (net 13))
 (segment (start 140.97 60.325) (end 140.97 56.515) (width 0.508) (layer F.Cu) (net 13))
 (segment (start 116.84 63.5) (end 123.825 63.5) (width 0.508) (layer F.Cu) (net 13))
 (segment (start 123.825 63.5) (end 125.73 61.595) (width 0.508) (layer F.Cu) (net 13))
 (segment (start 139.7 61.595) (end 140.97 60.325) (width 0.508) (layer F.Cu) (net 13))
 (segment (start 139.7 55.245) (end 137.16 55.245) (width 0.508) (layer F.Cu) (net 13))
 (segment (start 129.54 55.245) (end 128.27 56.515) (width 0.508) (layer F.Cu) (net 17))
 (segment (start 128.27 56.515) (end 128.27 58.26) (width 0.508) (layer F.Cu) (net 17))
 (segment (start 132.08 55.245) (end 132.08 56.99) (width 0.508) (layer F.Cu) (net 16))
 (segment (start 132.08 56.99) (end 130.81 58.26) (width 0.508) (layer F.Cu) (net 16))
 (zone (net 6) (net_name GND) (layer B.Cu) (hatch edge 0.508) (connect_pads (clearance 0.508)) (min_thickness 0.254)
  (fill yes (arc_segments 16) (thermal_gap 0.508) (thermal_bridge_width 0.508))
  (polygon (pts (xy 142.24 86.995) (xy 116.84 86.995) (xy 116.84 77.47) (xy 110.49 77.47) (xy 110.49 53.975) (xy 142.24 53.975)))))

